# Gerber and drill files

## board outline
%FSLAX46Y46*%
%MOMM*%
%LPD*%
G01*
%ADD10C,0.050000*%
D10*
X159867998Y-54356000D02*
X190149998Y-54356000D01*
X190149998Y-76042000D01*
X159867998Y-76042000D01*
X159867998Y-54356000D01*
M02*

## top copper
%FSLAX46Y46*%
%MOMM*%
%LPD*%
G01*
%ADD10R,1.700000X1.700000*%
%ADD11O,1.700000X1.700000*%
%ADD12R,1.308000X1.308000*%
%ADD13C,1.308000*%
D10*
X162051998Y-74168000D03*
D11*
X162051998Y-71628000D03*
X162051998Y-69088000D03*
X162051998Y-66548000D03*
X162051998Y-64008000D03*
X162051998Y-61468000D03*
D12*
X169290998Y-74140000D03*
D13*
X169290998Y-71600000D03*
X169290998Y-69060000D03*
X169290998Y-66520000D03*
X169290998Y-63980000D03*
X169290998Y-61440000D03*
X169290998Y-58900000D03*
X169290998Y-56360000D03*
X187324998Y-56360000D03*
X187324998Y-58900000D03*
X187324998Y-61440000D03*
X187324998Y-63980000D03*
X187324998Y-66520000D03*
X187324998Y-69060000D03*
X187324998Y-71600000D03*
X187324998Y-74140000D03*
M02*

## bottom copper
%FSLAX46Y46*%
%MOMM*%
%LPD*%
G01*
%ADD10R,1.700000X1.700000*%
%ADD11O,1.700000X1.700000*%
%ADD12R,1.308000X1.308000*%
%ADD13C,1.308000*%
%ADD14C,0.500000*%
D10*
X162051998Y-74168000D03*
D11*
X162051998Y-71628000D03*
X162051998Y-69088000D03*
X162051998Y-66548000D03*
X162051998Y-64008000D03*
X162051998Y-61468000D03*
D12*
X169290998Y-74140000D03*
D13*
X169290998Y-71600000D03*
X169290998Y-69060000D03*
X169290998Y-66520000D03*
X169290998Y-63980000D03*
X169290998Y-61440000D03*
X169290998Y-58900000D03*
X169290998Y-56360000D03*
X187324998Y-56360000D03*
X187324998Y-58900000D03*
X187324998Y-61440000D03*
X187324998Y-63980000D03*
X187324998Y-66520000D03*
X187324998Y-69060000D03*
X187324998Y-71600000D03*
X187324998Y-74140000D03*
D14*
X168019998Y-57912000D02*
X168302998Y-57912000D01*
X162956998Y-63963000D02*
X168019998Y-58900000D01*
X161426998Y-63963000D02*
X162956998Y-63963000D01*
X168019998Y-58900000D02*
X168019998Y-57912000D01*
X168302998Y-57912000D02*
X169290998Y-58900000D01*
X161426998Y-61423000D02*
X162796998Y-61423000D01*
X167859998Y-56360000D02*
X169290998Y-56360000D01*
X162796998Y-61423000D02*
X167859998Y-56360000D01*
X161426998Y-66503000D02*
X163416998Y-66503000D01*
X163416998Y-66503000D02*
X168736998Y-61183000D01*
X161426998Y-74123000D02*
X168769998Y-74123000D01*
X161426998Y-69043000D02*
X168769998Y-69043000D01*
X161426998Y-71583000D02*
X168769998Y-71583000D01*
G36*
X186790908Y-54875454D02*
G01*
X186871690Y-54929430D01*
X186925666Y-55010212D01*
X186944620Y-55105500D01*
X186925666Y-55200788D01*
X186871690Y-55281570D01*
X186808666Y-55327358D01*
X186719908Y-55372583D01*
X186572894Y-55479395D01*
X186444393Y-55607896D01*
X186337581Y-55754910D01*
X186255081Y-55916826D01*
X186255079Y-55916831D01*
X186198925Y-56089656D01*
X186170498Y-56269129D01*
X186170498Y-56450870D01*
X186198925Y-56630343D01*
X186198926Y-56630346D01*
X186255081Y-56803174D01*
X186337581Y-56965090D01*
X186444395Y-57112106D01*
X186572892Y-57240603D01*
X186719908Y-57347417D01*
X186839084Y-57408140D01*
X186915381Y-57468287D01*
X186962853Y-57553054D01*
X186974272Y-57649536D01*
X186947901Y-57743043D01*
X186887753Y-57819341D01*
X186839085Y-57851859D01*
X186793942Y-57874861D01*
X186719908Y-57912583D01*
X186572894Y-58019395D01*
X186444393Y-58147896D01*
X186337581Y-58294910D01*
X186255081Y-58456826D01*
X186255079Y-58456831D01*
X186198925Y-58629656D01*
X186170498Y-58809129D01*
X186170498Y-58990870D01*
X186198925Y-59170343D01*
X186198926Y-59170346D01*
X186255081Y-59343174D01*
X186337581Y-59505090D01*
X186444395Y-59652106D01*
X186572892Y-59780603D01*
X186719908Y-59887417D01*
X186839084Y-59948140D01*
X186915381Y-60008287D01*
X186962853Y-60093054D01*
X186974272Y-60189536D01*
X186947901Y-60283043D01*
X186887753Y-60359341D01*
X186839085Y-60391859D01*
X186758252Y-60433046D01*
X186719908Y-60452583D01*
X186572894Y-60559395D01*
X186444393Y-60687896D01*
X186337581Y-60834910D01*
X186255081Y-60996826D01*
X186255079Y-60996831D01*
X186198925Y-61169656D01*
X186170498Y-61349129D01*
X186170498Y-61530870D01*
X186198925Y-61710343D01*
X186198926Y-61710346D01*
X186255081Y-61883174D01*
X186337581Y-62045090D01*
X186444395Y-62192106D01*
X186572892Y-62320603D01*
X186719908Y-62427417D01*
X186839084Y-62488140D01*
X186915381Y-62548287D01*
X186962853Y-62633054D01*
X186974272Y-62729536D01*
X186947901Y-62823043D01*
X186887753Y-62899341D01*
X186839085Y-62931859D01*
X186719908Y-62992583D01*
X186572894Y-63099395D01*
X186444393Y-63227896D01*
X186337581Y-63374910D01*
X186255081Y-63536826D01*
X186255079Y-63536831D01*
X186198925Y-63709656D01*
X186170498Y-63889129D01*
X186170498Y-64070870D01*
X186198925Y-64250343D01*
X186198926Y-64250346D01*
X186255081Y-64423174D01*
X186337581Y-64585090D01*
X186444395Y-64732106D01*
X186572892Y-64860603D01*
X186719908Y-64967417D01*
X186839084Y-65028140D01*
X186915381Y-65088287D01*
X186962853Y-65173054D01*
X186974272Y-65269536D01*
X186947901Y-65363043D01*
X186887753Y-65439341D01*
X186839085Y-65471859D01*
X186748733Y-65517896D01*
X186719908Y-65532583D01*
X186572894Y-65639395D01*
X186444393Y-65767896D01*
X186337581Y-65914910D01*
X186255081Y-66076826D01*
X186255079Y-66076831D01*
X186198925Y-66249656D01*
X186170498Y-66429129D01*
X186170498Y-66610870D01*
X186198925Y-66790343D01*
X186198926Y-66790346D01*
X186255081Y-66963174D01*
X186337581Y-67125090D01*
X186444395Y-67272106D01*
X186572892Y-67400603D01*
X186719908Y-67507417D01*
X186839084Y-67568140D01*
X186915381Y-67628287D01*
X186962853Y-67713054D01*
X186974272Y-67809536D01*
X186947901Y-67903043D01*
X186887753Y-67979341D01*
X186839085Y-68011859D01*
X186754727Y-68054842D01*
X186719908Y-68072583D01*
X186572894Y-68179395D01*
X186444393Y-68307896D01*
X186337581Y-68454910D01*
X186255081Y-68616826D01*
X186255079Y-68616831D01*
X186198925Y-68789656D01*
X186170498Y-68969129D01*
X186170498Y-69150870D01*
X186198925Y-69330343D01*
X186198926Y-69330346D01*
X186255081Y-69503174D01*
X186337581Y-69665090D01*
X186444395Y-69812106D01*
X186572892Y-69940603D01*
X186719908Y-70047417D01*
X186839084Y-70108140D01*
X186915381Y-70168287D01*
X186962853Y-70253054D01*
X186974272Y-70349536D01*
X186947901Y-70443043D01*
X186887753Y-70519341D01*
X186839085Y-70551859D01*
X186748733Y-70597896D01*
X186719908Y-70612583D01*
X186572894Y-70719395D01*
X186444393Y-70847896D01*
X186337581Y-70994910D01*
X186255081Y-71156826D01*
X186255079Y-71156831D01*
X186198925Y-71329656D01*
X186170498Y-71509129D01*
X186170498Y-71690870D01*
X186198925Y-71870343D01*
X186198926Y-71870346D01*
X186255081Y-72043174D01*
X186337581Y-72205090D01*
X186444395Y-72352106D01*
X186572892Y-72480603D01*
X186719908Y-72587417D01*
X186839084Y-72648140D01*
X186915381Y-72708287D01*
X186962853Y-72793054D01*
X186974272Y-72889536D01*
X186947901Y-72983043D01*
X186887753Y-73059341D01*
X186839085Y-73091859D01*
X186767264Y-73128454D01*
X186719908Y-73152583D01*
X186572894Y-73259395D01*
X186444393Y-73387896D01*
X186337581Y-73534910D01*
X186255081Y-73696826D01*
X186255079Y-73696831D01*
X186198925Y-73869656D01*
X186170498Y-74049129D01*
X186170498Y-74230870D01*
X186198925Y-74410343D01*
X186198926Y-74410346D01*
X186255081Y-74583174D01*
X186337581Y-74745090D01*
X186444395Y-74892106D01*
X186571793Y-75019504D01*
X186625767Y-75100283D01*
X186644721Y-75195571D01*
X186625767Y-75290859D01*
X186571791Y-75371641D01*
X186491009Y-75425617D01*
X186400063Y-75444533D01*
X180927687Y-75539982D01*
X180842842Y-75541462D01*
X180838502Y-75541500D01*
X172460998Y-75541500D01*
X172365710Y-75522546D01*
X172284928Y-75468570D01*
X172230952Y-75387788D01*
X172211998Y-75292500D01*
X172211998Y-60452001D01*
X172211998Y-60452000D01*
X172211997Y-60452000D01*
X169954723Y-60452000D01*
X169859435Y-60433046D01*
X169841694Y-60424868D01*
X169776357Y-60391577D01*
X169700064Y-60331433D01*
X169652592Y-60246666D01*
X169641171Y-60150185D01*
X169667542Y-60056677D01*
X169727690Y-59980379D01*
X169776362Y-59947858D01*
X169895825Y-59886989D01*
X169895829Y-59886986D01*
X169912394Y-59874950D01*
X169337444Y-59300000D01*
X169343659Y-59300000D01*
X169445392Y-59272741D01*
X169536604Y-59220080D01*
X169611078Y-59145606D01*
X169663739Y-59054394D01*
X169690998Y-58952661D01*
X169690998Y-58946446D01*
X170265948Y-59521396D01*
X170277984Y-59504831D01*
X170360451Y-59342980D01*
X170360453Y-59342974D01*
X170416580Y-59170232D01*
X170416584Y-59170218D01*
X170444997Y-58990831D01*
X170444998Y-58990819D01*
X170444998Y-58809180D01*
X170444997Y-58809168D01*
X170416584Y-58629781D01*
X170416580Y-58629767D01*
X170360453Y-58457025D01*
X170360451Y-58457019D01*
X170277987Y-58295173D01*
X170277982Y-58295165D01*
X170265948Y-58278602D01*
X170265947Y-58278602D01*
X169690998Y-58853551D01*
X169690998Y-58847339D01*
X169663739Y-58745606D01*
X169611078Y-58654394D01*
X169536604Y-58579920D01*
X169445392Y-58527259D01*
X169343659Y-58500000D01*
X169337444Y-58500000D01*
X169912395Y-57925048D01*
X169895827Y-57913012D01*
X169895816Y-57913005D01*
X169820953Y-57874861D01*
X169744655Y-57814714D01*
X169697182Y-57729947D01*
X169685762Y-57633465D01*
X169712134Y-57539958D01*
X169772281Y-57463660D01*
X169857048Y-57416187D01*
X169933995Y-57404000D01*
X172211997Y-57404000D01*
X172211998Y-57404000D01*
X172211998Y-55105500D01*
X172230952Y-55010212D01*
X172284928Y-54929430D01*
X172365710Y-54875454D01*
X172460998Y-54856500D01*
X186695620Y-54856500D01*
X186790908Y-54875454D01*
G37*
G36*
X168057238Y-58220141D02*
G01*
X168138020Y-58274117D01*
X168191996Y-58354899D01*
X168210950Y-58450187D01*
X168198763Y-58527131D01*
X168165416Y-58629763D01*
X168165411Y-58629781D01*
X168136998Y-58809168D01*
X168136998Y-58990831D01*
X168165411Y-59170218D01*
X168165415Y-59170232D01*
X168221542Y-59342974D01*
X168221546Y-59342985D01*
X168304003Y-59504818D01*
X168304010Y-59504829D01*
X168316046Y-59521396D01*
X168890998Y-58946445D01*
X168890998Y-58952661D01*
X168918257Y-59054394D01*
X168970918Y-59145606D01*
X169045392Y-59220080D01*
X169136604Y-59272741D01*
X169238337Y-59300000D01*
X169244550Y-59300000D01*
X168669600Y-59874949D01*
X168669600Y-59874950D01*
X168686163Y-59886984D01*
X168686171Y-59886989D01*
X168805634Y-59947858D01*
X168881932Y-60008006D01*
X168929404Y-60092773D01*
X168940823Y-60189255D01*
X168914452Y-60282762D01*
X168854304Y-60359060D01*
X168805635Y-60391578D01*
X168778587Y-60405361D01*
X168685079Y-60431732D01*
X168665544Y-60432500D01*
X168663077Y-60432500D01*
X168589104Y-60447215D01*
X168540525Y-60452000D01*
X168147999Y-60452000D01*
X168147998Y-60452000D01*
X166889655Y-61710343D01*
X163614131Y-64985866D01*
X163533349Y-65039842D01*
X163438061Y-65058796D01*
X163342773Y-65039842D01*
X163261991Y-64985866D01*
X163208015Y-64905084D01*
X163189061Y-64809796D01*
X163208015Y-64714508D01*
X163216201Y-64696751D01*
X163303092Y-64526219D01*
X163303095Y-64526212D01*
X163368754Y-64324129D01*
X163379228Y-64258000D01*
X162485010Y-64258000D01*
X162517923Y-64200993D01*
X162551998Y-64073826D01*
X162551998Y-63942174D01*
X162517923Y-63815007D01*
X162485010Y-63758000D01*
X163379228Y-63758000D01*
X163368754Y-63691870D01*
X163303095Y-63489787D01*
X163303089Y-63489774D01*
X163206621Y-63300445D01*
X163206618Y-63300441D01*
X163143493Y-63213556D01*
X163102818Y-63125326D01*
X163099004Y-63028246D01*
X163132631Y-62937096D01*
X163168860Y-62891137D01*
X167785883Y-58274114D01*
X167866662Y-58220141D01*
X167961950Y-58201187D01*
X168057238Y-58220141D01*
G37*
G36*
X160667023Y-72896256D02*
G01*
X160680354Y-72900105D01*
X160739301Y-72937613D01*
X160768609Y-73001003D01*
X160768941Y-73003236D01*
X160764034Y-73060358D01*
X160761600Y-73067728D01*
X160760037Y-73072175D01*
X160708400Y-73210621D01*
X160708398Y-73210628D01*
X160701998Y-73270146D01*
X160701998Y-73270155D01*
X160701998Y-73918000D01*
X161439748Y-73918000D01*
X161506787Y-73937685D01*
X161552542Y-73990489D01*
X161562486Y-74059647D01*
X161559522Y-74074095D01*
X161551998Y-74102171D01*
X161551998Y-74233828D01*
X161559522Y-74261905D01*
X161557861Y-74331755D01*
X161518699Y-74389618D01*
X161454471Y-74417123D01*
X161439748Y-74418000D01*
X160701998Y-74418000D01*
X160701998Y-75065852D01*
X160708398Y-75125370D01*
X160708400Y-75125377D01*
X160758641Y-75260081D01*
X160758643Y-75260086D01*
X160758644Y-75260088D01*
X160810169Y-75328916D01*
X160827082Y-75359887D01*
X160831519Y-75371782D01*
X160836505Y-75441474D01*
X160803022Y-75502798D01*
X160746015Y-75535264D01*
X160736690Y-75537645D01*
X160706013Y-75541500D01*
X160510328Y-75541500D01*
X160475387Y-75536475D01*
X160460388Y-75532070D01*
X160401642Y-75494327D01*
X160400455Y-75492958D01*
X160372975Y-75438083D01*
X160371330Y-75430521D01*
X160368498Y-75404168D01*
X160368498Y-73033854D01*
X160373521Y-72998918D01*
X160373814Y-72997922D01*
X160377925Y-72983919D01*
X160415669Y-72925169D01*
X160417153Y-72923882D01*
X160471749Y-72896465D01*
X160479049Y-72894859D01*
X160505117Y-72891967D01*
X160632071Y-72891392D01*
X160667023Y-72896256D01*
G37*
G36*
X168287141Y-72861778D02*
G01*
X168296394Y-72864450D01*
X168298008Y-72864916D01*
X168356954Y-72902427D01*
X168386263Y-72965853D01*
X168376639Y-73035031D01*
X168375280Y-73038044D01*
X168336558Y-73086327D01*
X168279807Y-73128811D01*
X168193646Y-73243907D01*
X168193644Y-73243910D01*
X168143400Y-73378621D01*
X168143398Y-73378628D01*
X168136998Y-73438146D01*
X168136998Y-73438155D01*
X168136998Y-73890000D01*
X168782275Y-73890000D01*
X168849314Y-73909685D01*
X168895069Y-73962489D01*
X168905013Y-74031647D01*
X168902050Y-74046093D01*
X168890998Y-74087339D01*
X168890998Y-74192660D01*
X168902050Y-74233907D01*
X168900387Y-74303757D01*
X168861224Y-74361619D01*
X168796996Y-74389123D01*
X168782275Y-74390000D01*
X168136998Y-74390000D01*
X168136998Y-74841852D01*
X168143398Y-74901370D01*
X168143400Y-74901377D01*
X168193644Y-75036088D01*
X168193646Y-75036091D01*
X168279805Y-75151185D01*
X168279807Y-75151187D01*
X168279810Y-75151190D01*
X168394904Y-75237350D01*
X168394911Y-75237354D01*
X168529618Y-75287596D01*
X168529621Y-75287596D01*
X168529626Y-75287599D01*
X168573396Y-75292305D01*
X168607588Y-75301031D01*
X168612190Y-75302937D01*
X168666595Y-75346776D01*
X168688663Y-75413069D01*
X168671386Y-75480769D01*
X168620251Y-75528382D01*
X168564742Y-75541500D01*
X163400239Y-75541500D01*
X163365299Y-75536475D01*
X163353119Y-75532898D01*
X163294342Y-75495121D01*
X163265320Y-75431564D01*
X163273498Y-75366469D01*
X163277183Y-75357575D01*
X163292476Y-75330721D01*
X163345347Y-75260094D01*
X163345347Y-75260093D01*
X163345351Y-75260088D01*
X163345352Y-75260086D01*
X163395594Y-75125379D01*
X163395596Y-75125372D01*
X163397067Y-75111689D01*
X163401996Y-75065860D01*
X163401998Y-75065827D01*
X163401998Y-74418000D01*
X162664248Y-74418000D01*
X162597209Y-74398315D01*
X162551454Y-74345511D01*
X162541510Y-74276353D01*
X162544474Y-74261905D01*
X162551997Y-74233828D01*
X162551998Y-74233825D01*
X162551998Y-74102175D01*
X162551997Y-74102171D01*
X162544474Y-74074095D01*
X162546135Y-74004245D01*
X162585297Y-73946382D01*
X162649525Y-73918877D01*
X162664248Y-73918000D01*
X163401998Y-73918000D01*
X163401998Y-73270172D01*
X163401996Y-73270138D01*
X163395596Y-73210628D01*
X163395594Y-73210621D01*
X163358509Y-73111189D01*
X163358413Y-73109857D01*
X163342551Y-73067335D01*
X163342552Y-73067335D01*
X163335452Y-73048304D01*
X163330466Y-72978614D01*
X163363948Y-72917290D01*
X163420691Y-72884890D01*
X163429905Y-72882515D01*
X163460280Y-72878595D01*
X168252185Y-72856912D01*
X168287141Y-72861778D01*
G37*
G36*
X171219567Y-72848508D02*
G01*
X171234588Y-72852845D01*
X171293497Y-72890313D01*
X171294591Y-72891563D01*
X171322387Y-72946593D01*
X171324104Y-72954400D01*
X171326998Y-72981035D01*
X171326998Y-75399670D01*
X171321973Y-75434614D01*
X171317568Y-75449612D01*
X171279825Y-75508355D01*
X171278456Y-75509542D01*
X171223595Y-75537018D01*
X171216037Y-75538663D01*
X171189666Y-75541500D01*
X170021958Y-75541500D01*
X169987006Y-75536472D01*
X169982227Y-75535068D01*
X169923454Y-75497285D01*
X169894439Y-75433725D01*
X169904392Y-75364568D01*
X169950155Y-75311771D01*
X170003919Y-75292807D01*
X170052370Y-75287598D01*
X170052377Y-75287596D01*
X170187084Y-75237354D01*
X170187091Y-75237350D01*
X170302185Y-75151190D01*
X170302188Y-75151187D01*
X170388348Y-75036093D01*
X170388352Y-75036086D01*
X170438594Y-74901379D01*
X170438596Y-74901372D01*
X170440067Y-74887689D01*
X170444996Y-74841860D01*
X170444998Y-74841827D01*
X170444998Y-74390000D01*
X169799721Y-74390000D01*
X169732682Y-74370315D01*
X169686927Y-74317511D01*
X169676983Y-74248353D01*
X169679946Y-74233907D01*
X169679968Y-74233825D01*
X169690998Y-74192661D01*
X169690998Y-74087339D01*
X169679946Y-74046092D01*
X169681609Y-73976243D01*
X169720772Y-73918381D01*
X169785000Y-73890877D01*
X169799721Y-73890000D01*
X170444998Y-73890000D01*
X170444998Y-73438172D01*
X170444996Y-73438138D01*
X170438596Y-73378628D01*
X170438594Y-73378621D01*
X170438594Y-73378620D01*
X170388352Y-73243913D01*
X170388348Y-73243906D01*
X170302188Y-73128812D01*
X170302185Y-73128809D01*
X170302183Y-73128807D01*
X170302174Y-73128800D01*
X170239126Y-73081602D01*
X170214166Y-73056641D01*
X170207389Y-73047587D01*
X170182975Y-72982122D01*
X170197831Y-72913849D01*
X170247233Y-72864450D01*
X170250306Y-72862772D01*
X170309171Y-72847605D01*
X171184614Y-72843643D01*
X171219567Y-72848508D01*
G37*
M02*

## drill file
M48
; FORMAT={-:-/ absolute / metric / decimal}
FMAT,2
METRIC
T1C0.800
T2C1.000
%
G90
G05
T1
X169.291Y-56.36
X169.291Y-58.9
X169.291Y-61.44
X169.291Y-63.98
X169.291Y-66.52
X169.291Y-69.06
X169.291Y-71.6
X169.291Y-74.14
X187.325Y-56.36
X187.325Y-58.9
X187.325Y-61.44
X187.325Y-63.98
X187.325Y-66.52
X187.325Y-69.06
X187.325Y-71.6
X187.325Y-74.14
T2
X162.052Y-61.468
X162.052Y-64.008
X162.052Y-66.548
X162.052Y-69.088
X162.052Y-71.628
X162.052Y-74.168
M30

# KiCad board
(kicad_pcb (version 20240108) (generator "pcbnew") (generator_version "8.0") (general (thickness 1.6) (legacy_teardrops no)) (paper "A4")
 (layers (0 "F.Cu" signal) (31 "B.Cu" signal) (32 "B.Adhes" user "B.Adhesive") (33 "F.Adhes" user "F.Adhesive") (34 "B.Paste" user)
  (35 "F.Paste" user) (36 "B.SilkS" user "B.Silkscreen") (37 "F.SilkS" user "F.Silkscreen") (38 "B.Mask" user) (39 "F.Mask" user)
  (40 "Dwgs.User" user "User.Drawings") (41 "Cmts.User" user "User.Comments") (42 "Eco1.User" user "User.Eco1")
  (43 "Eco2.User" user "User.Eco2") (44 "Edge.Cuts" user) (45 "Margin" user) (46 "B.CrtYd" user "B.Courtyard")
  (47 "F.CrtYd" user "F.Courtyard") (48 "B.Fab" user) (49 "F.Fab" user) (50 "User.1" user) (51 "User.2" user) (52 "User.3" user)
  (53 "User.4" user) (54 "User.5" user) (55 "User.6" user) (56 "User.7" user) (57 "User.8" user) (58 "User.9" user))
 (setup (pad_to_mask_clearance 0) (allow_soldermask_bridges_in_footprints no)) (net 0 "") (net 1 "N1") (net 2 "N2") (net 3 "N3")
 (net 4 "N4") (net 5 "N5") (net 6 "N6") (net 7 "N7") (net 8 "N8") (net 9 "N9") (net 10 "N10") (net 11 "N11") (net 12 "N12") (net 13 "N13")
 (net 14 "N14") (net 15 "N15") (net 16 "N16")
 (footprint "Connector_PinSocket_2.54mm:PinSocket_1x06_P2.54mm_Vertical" (layer "F.Cu") (at 162.051998 74.168 180)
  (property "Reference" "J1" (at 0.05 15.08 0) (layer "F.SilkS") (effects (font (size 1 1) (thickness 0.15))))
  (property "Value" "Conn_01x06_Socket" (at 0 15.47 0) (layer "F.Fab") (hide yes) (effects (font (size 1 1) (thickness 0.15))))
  (pad "1" thru_hole rect (at 0 0 180) (size 1.7 1.7) (drill 1) (layers "*.Cu" "*.Mask") (remove_unused_layers no) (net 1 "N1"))
  (pad "2" thru_hole oval (at 0 2.54 180) (size 1.7 1.7) (drill 1) (layers "*.Cu" "*.Mask") (remove_unused_layers no) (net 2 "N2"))
  (pad "3" thru_hole oval (at 0 5.08 180) (size 1.7 1.7) (drill 1) (layers "*.Cu" "*.Mask") (remove_unused_layers no) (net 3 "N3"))
  (pad "4" thru_hole oval (at 0 7.62 180) (size 1.7 1.7) (drill 1) (layers "*.Cu" "*.Mask") (remove_unused_layers no) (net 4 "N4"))
  (pad "5" thru_hole oval (at 0 10.16 180) (size 1.7 1.7) (drill 1) (layers "*.Cu" "*.Mask") (remove_unused_layers no) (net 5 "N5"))
  (pad "6" thru_hole oval (at 0 12.7 180) (size 1.7 1.7) (drill 1) (layers "*.Cu" "*.Mask") (remove_unused_layers no) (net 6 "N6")))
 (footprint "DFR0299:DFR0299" (layer "F.Cu") (at 178.307998 65.25 180)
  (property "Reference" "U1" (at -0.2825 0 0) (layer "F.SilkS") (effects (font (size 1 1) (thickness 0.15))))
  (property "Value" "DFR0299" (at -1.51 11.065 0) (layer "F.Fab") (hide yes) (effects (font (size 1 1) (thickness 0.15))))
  (pad "1" thru_hole rect (at 9.017 -8.89 180) (size 1.308 1.308) (drill 0.8) (layers "*.Cu" "*.Mask") (remove_unused_layers no)
   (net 1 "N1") (solder_mask_margin 0.102))
  (pad "2" thru_hole circle (at 9.017 -6.35 180) (size 1.308 1.308) (drill 0.8) (layers "*.Cu" "*.Mask") (remove_unused_layers no)
   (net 2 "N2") (solder_mask_margin 0.102))
  (pad "3" thru_hole circle (at 9.017 -3.81 180) (size 1.308 1.308) (drill 0.8) (layers "*.Cu" "*.Mask") (remove_unused_layers no)
   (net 3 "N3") (solder_mask_margin 0.102))
  (pad "4" thru_hole circle (at 9.017 -1.27 180) (size 1.308 1.308) (drill 0.8) (layers "*.Cu" "*.Mask") (remove_unused_layers no)
   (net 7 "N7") (solder_mask_margin 0.102))
  (pad "5" thru_hole circle (at 9.017 1.27 180) (size 1.308 1.308) (drill 0.8) (layers "*.Cu" "*.Mask") (remove_unused_layers no)
   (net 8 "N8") (solder_mask_margin 0.102))
  (pad "6" thru_hole circle (at 9.017 3.81 180) (size 1.308 1.308) (drill 0.8) (layers "*.Cu" "*.Mask") (remove_unused_layers no)
   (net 4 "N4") (solder_mask_margin 0.102))
  (pad "7" thru_hole circle (at 9.017 6.35 180) (size 1.308 1.308) (drill 0.8) (layers "*.Cu" "*.Mask") (remove_unused_layers no)
   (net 5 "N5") (solder_mask_margin 0.102))
  (pad "8" thru_hole circle (at 9.017 8.89 180) (size 1.308 1.308) (drill 0.8) (layers "*.Cu" "*.Mask") (remove_unused_layers no)
   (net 6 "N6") (solder_mask_margin 0.102))
  (pad "9" thru_hole circle (at -9.017 8.89 180) (size 1.308 1.308) (drill 0.8) (layers "*.Cu" "*.Mask") (remove_unused_layers no)
   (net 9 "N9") (solder_mask_margin 0.102))
  (pad "10" thru_hole circle (at -9.017 6.35 180) (size 1.308 1.308) (drill 0.8) (layers "*.Cu" "*.Mask") (remove_unused_layers no)
   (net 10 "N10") (solder_mask_margin 0.102))
  (pad "11" thru_hole circle (at -9.017 3.81 180) (size 1.308 1.308) (drill 0.8) (layers "*.Cu" "*.Mask") (remove_unused_layers no)
   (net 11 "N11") (solder_mask_margin 0.102))
  (pad "12" thru_hole circle (at -9.017 1.27 180) (size 1.308 1.308) (drill 0.8) (layers "*.Cu" "*.Mask") (remove_unused_layers no)
   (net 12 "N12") (solder_mask_margin 0.102))
  (pad "13" thru_hole circle (at -9.017 -1.27 180) (size 1.308 1.308) (drill 0.8) (layers "*.Cu" "*.Mask") (remove_unused_layers no)
   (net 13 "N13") (solder_mask_margin 0.102))
  (pad "14" thru_hole circle (at -9.017 -3.81 180) (size 1.308 1.308) (drill 0.8) (layers "*.Cu" "*.Mask") (remove_unused_layers no)
   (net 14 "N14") (solder_mask_margin 0.102))
  (pad "15" thru_hole circle (at -9.017 -6.35 180) (size 1.308 1.308) (drill 0.8) (layers "*.Cu" "*.Mask") (remove_unused_layers no)
   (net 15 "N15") (solder_mask_margin 0.102))
  (pad "16" thru_hole circle (at -9.017 -8.89 180) (size 1.308 1.308) (drill 0.8) (layers "*.Cu" "*.Mask") (remove_unused_layers no)
   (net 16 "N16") (solder_mask_margin 0.102)))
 (gr_rect (start 159.867998 54.356) (end 190.149998 76.042) (stroke (width 0.05) (type default)) (fill none) (layer "Edge.Cuts"))
 (segment (start 168.019998 57.912) (end 168.302998 57.912) (width 0.5) (layer "B.Cu") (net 5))
 (segment (start 162.956998 63.963) (end 168.019998 58.9) (width 0.5) (layer "B.Cu") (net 5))
 (segment (start 161.426998 63.963) (end 162.956998 63.963) (width 0.5) (layer "B.Cu") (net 5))
 (segment (start 168.019998 58.9) (end 168.019998 57.912) (width 0.5) (layer "B.Cu") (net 5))
 (segment (start 168.302998 57.912) (end 169.290998 58.9) (width 0.5) (layer "B.Cu") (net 5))
 (segment (start 161.426998 61.423) (end 162.796998 61.423) (width 0.5) (layer "B.Cu") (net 6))
 (segment (start 167.859998 56.36) (end 169.290998 56.36) (width 0.5) (layer "B.Cu") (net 6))
 (segment (start 162.796998 61.423) (end 167.859998 56.36) (width 0.5) (layer "B.Cu") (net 6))
 (segment (start 161.426998 66.503) (end 163.416998 66.503) (width 0.5) (layer "B.Cu") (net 4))
 (segment (start 163.416998 66.503) (end 168.736998 61.183) (width 0.5) (layer "B.Cu") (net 4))
 (segment (start 161.426998 74.123) (end 168.769998 74.123) (width 0.5) (layer "B.Cu") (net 1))
 (segment (start 161.426998 69.043) (end 168.769998 69.043) (width 0.5) (layer "B.Cu") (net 3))
 (segment (start 161.426998 71.583) (end 168.769998 71.583) (width 0.5) (layer "B.Cu") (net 2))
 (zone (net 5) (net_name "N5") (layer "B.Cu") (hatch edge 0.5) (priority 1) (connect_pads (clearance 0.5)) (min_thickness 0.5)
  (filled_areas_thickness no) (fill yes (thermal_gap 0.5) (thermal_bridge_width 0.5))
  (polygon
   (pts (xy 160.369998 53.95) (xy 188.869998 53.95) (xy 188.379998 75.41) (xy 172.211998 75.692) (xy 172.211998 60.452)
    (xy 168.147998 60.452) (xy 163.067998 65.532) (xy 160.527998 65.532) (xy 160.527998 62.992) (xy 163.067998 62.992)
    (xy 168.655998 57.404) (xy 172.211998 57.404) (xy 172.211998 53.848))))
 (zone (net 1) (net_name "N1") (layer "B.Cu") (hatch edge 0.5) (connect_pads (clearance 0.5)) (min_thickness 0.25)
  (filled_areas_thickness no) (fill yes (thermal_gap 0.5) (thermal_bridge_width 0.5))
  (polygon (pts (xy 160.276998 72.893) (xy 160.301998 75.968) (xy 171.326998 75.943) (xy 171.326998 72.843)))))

